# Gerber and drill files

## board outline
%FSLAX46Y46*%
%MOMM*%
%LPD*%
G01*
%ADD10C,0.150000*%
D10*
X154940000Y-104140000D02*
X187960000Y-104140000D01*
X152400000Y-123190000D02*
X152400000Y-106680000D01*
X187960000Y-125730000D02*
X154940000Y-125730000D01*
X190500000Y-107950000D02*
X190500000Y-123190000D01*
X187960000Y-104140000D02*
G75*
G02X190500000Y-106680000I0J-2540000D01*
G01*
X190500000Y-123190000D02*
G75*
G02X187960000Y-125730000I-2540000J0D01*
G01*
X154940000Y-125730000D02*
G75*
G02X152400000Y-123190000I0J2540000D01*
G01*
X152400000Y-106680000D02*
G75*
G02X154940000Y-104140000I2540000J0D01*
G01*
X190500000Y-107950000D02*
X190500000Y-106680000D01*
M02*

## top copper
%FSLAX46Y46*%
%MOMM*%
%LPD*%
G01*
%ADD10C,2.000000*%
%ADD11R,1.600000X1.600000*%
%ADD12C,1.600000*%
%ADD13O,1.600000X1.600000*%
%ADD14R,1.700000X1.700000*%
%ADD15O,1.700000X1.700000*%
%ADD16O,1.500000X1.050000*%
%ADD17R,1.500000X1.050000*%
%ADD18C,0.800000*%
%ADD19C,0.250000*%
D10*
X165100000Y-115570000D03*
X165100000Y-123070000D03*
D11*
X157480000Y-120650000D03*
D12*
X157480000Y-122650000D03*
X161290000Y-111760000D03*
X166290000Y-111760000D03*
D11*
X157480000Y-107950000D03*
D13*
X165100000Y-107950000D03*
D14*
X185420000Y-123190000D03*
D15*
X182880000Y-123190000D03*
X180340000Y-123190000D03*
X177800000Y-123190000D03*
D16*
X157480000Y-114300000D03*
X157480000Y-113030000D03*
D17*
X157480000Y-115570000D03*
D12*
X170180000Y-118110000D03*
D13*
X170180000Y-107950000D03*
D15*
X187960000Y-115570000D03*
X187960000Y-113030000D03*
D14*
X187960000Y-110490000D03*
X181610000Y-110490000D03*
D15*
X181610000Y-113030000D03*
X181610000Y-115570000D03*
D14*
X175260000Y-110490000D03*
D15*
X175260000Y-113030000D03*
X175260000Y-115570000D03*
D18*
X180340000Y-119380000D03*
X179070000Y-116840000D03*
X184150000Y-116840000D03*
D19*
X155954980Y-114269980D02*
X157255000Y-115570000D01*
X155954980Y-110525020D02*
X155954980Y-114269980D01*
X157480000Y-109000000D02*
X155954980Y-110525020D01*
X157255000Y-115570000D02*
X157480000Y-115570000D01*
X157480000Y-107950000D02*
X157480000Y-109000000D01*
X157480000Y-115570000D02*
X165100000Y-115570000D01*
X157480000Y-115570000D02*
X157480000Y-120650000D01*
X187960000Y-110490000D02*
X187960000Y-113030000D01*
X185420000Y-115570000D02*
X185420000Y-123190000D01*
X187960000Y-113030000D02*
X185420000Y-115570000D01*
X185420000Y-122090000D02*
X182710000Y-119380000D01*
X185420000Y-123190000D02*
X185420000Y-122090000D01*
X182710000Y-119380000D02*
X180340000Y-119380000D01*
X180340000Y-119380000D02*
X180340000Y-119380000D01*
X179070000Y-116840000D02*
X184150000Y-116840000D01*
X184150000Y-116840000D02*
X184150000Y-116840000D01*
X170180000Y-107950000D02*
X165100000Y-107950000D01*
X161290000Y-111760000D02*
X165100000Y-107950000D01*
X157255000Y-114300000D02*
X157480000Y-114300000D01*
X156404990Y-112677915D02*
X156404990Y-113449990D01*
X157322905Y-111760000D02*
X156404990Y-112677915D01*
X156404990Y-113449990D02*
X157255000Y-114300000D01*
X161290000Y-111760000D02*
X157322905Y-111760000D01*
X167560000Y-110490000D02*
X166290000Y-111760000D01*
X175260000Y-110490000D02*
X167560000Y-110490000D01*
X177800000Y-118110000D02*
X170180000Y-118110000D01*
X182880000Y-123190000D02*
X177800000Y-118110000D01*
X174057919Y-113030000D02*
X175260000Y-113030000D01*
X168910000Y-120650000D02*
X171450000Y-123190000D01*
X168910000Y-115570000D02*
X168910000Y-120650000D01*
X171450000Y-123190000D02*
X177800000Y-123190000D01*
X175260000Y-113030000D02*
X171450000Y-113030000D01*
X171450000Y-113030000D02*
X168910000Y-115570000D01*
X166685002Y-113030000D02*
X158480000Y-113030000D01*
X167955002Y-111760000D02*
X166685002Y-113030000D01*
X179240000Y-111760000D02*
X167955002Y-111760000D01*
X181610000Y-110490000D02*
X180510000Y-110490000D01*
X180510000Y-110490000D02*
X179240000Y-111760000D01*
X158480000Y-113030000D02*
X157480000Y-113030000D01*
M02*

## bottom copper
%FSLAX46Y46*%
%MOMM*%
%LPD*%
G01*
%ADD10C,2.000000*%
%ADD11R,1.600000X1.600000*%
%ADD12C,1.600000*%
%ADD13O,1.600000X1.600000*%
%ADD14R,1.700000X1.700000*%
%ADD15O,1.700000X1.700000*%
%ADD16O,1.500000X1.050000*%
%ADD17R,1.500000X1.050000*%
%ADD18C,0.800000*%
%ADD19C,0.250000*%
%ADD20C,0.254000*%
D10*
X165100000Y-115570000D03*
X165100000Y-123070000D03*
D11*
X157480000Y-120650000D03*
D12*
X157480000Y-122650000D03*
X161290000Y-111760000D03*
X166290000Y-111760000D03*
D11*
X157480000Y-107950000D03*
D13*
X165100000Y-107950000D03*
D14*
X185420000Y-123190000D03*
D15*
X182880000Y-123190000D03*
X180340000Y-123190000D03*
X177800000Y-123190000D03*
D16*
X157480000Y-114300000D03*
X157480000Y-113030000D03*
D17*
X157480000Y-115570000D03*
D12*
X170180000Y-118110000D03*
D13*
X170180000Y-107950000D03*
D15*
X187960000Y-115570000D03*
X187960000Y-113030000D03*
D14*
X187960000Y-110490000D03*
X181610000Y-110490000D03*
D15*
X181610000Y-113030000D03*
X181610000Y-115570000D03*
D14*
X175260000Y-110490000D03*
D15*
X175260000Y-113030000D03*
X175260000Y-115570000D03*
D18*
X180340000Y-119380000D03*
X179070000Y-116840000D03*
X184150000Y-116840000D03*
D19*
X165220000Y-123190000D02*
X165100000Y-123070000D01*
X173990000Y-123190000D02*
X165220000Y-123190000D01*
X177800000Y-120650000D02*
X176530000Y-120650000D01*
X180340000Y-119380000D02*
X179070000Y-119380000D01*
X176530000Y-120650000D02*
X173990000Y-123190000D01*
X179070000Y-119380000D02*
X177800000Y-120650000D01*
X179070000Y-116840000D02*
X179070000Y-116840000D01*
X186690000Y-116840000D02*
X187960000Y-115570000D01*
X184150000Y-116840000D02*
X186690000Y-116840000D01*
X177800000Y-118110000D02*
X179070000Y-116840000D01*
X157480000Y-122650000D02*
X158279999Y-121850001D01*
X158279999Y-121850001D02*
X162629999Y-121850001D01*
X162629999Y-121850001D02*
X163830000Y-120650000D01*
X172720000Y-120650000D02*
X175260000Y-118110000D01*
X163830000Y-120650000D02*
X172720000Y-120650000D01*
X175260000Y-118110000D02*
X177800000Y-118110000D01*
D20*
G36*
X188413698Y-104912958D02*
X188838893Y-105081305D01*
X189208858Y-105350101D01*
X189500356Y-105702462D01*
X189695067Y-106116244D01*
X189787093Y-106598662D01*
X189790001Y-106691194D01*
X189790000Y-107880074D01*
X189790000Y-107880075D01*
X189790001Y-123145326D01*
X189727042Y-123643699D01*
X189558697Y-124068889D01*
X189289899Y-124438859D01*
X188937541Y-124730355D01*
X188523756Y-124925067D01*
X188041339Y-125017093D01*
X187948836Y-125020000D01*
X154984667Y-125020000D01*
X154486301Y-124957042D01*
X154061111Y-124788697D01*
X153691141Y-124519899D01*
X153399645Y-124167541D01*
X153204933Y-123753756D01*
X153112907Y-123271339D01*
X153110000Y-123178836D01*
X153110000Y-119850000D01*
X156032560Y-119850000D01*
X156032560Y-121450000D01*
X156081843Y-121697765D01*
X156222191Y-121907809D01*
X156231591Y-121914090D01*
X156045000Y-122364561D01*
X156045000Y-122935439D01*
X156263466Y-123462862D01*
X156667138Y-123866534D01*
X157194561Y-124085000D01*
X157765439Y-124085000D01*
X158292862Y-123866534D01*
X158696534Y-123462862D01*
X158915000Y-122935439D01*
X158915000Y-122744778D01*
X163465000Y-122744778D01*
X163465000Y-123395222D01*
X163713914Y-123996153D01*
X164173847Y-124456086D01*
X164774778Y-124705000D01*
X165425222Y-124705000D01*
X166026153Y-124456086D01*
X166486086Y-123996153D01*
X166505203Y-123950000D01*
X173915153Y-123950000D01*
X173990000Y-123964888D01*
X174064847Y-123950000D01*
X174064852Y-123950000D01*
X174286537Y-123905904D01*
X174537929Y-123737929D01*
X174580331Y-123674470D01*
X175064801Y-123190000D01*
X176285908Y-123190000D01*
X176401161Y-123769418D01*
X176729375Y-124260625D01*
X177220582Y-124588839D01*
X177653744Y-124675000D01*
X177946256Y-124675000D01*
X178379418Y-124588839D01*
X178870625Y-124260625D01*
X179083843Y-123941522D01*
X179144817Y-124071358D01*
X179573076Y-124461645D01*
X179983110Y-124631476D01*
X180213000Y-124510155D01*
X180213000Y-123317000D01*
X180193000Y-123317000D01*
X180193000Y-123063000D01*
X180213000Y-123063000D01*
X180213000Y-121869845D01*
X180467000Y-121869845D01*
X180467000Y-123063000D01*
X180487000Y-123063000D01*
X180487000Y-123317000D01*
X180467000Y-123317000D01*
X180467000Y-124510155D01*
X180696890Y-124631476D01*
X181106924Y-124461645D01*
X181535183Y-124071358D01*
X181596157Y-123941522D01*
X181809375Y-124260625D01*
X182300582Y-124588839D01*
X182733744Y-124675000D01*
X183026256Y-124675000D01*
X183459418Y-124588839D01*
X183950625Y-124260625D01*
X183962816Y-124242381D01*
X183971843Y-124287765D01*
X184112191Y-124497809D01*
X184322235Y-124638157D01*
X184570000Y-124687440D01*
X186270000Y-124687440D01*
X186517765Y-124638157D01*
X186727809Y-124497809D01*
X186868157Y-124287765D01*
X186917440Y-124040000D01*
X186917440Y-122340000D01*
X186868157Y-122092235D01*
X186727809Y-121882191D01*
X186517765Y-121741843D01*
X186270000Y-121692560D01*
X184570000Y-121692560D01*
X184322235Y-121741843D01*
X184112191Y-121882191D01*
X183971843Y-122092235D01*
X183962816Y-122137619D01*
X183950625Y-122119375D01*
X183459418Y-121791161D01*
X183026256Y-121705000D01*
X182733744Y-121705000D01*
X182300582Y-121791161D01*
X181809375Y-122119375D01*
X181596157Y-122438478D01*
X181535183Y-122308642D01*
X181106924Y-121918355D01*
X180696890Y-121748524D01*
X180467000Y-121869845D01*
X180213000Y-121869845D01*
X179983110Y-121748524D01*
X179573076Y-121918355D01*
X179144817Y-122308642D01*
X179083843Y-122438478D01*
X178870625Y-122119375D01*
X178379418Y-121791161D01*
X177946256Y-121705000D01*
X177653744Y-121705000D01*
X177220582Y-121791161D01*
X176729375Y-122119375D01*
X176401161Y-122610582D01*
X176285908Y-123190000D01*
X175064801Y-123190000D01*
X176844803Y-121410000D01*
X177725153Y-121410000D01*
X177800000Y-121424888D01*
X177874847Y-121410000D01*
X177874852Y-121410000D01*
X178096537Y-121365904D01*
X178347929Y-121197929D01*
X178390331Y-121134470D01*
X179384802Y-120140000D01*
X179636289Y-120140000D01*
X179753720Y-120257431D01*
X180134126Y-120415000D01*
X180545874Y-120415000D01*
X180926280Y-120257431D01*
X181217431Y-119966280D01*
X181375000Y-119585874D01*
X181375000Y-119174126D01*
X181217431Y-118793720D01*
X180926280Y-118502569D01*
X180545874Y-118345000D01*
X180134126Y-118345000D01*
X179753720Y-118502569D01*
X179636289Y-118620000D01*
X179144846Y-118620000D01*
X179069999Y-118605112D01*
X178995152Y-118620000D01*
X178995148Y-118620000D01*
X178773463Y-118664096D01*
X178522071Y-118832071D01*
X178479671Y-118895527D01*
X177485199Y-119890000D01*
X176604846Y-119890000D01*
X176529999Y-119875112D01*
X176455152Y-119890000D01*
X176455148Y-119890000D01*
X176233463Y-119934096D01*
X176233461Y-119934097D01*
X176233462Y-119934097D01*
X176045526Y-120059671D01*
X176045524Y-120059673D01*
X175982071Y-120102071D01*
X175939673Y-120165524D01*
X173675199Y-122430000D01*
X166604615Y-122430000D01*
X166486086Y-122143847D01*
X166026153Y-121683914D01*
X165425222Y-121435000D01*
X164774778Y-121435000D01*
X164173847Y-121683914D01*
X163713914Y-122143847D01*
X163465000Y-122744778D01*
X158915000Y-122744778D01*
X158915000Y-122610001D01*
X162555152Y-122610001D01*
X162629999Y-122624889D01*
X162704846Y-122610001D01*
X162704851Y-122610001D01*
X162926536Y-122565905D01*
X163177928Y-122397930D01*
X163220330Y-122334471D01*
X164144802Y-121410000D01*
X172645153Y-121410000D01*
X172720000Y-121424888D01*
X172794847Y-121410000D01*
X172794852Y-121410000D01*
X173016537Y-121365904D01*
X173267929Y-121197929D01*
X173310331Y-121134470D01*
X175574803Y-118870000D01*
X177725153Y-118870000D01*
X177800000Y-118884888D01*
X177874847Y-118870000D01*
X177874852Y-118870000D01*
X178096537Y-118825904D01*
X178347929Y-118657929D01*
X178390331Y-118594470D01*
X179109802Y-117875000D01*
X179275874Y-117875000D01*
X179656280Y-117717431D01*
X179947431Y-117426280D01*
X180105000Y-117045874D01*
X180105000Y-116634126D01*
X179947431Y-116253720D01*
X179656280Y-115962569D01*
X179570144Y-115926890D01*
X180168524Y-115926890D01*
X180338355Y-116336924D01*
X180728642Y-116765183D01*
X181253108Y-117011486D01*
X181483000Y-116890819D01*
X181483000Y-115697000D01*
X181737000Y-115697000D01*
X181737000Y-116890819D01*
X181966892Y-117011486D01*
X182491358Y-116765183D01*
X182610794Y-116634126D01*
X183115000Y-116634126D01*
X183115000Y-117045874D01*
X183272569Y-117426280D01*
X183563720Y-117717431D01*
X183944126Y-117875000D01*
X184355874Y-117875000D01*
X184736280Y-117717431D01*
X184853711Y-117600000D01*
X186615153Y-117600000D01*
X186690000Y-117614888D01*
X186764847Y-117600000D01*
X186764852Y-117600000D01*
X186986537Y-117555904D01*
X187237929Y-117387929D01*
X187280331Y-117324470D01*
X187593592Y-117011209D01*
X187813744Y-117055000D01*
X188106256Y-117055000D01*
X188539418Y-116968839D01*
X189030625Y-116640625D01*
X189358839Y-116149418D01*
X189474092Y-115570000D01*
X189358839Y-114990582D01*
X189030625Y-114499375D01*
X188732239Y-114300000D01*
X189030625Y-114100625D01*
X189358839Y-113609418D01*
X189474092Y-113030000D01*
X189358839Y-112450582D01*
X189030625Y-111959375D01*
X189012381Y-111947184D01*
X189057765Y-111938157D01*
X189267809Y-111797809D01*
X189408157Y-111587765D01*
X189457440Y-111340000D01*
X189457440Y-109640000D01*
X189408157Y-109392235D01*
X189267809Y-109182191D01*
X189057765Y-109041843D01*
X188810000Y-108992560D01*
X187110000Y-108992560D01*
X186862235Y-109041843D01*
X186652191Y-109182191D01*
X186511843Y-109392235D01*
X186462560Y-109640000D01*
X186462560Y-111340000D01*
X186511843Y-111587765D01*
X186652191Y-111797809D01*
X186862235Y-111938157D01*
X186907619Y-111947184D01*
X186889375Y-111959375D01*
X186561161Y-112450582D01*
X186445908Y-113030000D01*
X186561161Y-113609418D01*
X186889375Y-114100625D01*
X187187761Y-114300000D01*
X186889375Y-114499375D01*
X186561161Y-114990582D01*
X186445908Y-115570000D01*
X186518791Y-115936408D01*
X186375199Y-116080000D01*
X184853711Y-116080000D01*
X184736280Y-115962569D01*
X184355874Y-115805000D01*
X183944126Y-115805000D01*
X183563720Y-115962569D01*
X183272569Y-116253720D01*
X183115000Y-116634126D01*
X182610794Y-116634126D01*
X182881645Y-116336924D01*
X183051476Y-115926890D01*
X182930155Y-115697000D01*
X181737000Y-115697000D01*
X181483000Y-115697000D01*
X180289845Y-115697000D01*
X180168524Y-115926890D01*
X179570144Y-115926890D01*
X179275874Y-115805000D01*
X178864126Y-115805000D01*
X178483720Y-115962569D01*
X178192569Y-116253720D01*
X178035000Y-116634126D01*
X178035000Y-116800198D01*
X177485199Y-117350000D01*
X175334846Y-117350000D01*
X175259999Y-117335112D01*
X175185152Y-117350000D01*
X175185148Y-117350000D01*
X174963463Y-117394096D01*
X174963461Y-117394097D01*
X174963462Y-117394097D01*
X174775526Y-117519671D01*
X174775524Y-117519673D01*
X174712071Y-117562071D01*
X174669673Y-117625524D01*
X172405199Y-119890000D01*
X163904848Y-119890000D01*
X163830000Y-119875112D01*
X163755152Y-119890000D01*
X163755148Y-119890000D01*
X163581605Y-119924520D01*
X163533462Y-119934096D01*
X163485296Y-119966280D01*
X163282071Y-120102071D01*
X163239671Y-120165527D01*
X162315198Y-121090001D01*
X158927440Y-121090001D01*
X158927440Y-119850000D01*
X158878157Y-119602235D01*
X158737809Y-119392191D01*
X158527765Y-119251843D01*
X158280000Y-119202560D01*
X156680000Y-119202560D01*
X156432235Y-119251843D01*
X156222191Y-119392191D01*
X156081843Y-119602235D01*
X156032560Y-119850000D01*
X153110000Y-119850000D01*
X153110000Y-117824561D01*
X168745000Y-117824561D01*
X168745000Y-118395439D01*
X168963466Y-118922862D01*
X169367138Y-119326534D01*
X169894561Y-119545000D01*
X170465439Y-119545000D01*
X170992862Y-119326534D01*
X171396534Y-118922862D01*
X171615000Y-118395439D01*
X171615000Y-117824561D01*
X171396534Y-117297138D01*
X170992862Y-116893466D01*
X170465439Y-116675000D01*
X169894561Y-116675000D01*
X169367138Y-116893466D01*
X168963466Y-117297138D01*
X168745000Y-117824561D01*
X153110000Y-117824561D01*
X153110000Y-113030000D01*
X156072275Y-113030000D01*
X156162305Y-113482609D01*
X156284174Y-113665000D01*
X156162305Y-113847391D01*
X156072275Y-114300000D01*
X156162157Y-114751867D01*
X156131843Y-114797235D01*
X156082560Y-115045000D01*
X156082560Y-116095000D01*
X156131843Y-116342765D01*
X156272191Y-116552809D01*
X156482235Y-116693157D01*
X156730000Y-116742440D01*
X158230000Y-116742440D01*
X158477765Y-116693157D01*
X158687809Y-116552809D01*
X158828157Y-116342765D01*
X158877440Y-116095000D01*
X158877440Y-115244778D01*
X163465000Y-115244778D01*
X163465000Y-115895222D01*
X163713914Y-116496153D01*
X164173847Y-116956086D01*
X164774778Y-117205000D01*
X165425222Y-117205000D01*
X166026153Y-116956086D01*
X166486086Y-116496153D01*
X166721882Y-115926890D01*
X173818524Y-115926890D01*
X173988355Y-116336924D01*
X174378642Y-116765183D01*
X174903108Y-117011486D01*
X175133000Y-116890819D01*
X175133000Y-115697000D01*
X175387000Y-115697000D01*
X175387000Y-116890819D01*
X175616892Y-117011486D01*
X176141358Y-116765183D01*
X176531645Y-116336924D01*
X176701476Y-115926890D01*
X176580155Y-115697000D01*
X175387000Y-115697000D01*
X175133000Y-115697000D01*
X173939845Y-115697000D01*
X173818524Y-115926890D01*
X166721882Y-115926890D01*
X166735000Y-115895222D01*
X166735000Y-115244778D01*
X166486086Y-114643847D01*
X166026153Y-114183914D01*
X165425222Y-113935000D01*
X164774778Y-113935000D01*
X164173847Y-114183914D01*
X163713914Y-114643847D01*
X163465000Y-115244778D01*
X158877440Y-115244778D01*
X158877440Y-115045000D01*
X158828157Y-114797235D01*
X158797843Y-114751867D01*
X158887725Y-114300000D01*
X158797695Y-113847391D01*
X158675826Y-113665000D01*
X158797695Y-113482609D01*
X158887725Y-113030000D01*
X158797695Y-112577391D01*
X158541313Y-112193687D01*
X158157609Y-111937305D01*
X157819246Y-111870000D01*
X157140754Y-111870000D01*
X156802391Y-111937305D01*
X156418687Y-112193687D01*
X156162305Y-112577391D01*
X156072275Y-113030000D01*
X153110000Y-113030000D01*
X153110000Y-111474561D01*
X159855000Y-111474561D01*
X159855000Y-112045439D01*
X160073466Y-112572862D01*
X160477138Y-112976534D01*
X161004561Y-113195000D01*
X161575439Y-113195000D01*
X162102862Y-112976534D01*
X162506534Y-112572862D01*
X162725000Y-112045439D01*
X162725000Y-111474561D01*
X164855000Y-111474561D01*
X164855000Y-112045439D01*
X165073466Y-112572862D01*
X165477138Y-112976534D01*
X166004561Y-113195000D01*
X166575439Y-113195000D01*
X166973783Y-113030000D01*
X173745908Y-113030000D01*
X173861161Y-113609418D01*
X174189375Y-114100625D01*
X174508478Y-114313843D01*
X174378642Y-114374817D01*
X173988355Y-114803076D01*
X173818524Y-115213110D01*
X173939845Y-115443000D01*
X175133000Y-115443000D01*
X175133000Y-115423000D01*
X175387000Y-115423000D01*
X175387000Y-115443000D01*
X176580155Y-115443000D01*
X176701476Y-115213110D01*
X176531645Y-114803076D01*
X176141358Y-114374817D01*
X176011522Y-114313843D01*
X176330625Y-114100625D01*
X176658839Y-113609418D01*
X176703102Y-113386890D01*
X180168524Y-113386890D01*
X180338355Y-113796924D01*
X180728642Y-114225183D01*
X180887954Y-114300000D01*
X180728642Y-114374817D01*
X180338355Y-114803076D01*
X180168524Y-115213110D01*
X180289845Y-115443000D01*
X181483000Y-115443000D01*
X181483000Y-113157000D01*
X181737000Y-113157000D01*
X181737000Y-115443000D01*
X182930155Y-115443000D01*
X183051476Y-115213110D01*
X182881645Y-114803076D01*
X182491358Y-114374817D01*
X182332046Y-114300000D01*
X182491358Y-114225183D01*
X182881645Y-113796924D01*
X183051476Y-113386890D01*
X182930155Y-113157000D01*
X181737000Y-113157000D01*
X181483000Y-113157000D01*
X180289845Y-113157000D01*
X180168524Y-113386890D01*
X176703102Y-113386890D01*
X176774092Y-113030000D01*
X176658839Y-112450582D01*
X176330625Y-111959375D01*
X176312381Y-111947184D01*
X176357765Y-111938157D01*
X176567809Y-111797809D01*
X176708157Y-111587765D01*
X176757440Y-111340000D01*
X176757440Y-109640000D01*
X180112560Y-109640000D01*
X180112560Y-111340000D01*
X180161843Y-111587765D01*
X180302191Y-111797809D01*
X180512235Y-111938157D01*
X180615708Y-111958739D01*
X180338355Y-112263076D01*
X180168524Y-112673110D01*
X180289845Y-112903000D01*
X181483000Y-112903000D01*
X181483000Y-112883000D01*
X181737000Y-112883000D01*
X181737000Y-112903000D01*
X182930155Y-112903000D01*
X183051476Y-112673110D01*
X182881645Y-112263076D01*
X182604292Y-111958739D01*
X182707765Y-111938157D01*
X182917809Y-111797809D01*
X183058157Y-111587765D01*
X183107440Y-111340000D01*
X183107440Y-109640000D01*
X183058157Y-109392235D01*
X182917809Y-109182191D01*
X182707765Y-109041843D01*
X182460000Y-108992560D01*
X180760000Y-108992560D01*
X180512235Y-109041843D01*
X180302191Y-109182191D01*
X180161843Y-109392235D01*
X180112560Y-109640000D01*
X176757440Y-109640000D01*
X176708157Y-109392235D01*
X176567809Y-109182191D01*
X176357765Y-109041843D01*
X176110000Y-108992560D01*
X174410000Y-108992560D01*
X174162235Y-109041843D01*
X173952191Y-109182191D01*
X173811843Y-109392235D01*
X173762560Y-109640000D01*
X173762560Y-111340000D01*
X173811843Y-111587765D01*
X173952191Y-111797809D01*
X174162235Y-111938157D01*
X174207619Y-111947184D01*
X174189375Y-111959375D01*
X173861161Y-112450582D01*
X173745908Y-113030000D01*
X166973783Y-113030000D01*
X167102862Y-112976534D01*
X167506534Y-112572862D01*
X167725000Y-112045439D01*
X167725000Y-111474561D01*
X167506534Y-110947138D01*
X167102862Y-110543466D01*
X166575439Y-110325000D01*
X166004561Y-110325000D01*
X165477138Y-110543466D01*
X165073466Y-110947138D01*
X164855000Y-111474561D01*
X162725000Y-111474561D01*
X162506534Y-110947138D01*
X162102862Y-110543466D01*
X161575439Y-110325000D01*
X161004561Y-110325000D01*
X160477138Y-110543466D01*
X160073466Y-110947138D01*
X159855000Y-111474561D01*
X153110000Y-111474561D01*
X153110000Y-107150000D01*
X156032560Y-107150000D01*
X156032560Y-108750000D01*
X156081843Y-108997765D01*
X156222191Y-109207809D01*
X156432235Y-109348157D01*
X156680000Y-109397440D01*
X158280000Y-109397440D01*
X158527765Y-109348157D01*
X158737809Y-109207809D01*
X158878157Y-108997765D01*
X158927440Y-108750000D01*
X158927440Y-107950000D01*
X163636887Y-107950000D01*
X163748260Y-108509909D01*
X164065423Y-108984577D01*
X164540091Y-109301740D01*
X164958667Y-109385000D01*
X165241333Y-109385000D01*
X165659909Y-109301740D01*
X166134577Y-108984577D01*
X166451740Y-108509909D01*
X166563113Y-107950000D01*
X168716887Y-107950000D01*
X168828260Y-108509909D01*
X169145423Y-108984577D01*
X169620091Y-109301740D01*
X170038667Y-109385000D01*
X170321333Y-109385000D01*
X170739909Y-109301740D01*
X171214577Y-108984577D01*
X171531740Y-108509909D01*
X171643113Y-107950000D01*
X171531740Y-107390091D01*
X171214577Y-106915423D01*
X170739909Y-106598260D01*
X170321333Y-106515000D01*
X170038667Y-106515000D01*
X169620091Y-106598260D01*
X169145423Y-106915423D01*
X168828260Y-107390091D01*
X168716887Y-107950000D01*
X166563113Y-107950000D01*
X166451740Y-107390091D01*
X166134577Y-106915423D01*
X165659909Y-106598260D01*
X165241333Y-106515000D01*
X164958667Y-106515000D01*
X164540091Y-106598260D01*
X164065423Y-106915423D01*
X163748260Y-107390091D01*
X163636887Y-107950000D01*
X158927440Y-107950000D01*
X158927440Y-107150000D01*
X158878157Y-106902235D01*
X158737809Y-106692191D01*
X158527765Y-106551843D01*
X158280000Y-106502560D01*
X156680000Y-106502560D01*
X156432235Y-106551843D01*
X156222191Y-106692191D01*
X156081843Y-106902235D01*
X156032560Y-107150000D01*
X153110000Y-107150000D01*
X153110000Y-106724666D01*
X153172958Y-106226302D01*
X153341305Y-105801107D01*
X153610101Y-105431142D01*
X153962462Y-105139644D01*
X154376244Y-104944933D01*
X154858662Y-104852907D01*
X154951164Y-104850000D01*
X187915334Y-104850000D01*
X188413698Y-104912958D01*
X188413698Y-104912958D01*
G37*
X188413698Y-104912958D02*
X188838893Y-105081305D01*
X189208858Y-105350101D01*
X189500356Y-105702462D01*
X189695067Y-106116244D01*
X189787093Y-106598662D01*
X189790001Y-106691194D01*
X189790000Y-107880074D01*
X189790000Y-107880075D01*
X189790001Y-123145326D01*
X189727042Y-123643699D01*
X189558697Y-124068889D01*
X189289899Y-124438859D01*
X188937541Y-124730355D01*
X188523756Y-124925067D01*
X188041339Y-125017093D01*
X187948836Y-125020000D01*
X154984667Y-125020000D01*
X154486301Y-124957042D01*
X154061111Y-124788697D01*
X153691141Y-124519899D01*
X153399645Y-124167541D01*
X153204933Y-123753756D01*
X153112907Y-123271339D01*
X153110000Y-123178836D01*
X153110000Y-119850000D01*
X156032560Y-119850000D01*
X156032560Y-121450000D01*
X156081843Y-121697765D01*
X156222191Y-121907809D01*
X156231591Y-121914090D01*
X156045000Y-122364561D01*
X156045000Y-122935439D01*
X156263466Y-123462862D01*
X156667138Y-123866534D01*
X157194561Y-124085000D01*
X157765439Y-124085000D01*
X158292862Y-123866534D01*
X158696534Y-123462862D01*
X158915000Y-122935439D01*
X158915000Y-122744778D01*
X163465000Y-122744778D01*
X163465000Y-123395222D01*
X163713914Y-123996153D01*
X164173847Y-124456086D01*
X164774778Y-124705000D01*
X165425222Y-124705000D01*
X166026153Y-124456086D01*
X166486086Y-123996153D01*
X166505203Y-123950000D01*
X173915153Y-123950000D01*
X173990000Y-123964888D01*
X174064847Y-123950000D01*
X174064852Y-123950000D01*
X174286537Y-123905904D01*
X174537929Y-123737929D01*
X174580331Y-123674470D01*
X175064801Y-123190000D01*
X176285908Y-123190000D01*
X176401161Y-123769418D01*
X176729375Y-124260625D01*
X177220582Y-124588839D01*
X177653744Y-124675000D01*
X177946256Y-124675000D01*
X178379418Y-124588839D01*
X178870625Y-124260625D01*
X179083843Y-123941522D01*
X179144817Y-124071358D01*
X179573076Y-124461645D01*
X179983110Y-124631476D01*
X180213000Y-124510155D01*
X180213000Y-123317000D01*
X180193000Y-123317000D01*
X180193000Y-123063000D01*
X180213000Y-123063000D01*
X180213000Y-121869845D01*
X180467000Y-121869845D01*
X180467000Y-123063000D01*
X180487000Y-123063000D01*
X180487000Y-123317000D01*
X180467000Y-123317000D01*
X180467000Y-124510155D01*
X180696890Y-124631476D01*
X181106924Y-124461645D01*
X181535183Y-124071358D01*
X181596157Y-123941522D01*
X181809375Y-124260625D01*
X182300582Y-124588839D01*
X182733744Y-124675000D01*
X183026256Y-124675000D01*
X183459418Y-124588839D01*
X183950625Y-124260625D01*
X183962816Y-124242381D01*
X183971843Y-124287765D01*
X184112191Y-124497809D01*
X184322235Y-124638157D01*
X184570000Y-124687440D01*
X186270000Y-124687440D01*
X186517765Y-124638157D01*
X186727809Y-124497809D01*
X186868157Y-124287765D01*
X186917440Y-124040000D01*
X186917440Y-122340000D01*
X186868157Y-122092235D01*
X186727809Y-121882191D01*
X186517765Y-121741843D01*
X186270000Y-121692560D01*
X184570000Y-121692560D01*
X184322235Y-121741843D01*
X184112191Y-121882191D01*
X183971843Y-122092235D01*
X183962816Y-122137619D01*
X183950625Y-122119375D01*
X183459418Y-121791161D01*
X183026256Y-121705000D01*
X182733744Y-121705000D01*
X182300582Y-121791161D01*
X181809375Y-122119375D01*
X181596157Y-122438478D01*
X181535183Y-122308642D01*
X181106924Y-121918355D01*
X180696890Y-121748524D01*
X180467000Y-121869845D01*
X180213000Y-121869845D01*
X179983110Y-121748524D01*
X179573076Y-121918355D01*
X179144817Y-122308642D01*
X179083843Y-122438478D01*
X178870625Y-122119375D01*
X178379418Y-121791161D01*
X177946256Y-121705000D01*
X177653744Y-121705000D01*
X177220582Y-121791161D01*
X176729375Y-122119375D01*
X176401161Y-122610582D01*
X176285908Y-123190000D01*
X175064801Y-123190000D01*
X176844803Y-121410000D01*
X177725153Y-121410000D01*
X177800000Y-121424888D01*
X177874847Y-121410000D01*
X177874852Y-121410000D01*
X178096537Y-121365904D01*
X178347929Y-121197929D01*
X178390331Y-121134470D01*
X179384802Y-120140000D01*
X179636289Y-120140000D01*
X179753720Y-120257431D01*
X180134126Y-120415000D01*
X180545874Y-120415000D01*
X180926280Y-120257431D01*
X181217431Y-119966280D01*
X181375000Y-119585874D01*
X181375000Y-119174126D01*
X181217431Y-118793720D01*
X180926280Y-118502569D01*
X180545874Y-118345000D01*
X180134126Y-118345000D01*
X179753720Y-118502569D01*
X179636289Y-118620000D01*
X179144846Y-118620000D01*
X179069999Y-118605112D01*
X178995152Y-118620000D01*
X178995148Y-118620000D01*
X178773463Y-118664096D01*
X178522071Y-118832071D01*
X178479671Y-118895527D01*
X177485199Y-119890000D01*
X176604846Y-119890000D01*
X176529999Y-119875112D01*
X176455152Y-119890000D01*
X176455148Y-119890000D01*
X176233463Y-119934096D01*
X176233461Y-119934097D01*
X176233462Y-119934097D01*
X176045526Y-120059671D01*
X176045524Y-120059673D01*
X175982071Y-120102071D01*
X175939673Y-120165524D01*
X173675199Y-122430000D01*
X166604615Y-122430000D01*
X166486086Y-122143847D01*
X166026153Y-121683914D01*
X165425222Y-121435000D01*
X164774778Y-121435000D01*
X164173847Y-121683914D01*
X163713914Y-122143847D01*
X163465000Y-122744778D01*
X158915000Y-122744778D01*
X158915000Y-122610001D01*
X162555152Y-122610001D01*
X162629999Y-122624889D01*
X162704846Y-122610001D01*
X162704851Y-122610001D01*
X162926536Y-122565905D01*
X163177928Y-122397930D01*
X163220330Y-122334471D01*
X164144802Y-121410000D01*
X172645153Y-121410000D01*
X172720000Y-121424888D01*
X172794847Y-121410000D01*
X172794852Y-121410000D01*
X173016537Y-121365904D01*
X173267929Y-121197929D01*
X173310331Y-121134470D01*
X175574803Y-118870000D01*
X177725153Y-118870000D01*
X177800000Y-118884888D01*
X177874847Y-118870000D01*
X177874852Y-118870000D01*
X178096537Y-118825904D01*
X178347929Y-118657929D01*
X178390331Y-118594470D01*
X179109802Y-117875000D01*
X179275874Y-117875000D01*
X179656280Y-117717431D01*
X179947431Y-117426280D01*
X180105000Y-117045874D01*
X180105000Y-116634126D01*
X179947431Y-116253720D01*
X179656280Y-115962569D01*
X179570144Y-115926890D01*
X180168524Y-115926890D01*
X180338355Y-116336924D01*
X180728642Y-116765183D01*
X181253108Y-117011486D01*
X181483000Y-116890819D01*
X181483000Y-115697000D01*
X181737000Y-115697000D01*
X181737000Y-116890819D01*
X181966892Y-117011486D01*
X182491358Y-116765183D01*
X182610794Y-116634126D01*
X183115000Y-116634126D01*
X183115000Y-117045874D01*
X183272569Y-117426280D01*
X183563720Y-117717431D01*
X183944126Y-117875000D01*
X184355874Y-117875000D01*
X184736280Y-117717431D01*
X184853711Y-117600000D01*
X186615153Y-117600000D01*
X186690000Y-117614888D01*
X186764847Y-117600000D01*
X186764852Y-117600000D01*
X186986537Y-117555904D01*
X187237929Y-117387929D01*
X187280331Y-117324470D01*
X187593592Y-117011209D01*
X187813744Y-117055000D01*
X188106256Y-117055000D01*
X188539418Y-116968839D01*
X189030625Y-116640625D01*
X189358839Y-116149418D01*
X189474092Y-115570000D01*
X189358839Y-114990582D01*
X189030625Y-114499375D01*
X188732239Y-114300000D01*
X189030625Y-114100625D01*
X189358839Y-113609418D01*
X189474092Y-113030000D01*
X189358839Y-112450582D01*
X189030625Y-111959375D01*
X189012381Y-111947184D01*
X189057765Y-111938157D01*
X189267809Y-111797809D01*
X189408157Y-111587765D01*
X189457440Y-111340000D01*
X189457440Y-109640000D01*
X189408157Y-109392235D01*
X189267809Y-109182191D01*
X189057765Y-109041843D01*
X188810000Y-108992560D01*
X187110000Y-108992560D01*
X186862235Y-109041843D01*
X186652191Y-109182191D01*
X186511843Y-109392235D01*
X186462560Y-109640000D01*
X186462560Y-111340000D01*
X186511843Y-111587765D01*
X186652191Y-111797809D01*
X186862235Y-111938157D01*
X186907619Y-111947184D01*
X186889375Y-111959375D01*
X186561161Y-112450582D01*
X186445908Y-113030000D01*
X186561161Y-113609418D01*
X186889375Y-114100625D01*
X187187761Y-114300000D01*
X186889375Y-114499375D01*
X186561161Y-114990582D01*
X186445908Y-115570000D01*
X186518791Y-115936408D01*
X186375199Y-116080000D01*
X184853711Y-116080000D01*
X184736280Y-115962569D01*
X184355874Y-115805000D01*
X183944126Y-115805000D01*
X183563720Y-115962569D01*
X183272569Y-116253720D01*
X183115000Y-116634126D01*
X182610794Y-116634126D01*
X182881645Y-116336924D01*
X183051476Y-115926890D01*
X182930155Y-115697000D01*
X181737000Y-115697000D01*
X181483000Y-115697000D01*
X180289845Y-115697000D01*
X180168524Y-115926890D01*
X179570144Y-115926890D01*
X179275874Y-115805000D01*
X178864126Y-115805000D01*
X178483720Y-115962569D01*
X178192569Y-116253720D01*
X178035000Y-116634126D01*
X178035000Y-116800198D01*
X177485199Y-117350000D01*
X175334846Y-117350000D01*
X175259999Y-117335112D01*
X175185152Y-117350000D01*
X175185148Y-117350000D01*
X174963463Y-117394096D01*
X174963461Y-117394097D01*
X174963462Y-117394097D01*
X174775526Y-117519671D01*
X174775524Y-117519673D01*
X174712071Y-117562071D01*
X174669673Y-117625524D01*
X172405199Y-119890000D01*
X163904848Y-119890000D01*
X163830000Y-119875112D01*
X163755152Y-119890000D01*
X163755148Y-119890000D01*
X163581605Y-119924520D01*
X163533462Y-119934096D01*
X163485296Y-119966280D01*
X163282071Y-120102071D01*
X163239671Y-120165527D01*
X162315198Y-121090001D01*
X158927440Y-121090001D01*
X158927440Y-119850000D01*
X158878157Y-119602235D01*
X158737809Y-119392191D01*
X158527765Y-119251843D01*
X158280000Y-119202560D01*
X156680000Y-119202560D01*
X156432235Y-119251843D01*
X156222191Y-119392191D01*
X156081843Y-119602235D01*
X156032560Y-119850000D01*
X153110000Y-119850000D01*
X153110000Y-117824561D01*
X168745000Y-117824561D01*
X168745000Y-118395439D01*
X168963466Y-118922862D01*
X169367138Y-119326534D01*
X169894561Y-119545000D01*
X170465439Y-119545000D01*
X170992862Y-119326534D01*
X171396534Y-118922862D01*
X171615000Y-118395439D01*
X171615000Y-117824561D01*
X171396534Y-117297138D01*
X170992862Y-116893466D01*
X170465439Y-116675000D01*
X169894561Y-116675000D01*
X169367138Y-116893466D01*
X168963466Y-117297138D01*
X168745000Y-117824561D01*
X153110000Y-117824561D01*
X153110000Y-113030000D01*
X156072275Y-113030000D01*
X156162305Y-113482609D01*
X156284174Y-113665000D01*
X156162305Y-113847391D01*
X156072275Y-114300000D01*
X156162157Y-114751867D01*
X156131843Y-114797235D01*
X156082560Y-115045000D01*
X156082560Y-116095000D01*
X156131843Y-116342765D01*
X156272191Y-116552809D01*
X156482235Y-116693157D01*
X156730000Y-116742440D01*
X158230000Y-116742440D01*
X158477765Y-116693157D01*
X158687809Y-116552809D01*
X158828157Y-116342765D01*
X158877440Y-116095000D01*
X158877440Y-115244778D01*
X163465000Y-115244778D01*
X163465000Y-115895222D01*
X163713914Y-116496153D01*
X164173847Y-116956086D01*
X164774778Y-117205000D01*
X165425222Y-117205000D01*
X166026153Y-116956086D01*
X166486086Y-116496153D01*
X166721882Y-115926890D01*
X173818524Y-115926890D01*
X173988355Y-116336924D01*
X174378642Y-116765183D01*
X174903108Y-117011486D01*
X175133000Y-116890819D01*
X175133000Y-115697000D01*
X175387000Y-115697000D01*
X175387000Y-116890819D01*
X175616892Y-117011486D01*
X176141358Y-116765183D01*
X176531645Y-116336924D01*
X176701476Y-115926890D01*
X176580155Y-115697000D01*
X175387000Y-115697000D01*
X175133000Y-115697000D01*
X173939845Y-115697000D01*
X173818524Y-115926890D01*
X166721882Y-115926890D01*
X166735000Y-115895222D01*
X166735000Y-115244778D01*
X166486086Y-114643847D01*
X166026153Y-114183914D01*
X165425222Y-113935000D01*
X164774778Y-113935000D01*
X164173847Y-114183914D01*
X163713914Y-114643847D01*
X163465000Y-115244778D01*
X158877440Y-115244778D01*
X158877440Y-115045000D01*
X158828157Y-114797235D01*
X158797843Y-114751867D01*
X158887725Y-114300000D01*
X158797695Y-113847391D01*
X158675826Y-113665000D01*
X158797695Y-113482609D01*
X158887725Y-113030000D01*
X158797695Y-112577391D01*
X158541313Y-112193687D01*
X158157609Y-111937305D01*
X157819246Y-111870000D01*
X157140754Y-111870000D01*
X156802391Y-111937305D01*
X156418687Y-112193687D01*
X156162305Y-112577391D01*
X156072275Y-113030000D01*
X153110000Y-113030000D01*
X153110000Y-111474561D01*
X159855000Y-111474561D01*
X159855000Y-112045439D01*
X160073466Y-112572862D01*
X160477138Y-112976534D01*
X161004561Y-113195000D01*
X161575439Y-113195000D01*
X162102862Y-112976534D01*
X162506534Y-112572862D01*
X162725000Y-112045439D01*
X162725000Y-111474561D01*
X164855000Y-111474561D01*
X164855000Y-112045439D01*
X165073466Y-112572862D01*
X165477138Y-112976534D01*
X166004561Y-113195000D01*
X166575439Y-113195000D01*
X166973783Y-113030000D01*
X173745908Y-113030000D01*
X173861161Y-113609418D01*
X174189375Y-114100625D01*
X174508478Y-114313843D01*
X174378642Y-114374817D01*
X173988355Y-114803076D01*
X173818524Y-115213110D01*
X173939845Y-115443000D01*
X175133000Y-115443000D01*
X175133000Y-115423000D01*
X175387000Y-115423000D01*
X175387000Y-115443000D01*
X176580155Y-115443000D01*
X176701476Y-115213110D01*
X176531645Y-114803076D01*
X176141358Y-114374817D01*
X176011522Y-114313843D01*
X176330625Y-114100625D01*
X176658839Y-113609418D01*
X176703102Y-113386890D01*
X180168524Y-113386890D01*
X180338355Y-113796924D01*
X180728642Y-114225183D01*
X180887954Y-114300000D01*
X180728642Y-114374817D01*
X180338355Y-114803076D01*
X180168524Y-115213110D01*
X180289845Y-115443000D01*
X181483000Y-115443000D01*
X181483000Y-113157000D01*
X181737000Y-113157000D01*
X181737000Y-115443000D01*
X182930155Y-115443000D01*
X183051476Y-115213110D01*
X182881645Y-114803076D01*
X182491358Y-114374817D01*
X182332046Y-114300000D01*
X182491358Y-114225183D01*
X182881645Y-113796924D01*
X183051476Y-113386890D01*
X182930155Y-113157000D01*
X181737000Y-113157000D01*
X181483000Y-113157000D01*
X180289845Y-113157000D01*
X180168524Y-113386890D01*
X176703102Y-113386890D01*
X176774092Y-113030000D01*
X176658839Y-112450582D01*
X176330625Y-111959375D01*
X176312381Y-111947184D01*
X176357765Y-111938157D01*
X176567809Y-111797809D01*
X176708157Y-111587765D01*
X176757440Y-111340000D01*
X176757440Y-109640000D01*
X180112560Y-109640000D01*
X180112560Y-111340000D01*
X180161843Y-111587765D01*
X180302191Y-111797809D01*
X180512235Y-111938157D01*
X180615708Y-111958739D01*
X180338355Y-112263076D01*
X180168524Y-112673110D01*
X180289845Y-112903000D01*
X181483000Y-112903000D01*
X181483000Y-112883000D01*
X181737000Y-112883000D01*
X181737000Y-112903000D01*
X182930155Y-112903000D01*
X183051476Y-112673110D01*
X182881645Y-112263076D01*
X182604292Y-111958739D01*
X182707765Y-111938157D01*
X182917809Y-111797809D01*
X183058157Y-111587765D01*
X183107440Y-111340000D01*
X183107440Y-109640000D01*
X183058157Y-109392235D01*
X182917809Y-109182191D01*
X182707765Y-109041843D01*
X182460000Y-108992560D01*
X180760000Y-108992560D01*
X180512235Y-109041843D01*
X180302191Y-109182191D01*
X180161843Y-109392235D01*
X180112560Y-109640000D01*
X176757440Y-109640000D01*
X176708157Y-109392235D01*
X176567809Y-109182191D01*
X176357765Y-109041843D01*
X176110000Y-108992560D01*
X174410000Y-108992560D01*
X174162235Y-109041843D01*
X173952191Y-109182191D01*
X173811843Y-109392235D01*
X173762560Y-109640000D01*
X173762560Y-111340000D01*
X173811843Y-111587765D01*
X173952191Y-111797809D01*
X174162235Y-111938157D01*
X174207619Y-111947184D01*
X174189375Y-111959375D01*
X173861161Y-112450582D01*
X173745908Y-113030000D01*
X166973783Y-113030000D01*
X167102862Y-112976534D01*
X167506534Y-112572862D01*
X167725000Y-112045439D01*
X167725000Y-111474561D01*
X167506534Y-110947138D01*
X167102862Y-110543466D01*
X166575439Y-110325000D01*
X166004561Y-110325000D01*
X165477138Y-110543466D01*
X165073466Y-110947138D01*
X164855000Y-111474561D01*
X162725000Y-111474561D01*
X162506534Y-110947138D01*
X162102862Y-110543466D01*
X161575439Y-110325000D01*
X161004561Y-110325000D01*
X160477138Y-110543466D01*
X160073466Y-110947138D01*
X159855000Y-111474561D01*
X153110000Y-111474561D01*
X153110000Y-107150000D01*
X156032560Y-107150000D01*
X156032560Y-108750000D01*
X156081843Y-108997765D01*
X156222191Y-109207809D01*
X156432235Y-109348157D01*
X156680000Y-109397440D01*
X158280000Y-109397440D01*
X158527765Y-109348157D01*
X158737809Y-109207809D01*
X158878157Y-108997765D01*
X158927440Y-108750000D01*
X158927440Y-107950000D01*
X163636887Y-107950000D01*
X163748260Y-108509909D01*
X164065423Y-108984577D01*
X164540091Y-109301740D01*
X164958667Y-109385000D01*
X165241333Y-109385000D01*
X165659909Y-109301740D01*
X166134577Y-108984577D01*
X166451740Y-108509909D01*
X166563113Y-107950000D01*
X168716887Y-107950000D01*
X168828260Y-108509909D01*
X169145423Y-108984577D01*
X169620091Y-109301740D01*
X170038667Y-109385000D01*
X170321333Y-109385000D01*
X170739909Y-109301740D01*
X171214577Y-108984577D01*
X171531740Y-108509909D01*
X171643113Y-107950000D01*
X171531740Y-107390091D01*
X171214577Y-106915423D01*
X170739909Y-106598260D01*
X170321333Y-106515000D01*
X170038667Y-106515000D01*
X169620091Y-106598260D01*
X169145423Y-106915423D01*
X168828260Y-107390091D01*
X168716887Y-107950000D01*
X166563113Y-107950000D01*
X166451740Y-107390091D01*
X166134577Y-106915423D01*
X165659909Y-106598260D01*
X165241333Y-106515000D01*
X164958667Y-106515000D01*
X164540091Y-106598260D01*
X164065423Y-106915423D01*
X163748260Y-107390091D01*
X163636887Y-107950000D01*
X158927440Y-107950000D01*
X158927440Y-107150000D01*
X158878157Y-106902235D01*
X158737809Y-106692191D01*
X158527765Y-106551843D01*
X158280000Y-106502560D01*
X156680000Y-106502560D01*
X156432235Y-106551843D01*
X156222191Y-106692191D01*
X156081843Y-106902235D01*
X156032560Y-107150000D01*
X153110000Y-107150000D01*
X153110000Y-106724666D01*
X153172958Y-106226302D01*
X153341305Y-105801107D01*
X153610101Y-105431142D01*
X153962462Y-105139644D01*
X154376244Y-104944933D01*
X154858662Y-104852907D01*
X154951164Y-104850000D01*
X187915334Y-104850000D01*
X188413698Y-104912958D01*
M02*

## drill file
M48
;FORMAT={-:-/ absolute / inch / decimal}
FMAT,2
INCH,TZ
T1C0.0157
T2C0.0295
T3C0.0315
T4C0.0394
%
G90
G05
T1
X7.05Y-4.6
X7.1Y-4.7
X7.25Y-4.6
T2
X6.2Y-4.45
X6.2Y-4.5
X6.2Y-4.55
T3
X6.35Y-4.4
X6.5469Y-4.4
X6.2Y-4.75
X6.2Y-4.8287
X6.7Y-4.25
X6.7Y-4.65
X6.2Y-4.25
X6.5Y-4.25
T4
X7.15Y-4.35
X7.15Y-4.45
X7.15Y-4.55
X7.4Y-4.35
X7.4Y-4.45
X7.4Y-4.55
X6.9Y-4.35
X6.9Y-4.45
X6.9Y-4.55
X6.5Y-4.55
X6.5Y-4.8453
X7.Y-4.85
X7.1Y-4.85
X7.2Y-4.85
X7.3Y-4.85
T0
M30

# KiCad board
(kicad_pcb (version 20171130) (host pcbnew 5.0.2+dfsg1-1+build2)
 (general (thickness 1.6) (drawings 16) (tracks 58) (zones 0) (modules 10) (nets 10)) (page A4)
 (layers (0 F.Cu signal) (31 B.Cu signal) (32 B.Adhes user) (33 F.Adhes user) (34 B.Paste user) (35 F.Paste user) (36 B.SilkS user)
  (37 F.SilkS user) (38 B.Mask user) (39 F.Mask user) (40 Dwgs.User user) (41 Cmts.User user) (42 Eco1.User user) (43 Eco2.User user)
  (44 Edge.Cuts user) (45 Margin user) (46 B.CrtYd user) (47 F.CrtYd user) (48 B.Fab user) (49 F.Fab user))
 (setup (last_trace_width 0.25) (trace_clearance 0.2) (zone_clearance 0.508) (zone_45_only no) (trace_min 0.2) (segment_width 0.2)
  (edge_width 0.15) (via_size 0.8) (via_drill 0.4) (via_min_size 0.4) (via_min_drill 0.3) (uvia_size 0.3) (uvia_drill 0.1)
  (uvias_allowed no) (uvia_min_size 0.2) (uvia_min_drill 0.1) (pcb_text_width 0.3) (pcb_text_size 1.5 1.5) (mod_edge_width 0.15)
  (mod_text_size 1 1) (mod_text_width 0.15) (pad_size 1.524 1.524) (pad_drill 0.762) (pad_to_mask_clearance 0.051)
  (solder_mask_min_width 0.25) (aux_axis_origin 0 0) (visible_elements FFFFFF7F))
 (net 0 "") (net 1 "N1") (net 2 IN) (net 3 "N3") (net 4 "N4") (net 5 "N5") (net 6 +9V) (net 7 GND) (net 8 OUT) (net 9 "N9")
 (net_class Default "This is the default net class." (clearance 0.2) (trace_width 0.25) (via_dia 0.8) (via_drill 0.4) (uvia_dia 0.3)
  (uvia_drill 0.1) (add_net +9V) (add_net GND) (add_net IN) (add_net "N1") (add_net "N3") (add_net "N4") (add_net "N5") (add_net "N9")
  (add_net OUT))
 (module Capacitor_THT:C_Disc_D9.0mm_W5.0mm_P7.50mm (layer F.Cu) (at 165.1 115.57 270)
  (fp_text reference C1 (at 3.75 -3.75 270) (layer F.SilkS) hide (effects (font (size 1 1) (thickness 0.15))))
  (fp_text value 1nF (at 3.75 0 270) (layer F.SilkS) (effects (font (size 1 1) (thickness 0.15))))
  (pad 1 thru_hole circle (at 0 0 270) (size 2 2) (drill 1) (layers *.Cu *.Mask) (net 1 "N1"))
  (pad 2 thru_hole circle (at 7.5 0 270) (size 2 2) (drill 1) (layers *.Cu *.Mask) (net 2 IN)))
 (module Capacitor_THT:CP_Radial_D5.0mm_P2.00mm (layer F.Cu) (at 157.48 120.65 270)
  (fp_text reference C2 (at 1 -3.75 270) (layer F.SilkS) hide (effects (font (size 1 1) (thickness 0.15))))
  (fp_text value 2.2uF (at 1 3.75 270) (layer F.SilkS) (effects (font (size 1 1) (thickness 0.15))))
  (pad 1 thru_hole rect (at 0 0 270) (size 1.6 1.6) (drill 0.8) (layers *.Cu *.Mask) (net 1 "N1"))
  (pad 2 thru_hole circle (at 2 0 270) (size 1.6 1.6) (drill 0.8) (layers *.Cu *.Mask) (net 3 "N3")))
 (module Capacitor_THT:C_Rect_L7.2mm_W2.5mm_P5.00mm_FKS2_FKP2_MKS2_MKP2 (layer F.Cu) (at 161.29 111.76)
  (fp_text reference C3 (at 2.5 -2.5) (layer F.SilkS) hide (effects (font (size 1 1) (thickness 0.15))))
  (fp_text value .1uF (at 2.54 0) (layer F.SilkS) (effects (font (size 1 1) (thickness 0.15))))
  (pad 1 thru_hole circle (at 0 0) (size 1.6 1.6) (drill 0.8) (layers *.Cu *.Mask) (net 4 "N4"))
  (pad 2 thru_hole circle (at 5 0) (size 1.6 1.6) (drill 0.8) (layers *.Cu *.Mask) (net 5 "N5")))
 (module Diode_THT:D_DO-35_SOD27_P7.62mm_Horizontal (layer F.Cu) (at 157.48 107.95)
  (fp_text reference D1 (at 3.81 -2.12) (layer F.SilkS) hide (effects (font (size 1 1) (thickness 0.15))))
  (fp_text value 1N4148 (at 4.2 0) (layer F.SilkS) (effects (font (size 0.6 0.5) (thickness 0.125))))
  (pad 1 thru_hole rect (at 0 0) (size 1.6 1.6) (drill 0.8) (layers *.Cu *.Mask) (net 1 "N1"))
  (pad 2 thru_hole oval (at 7.62 0) (size 1.6 1.6) (drill 0.8) (layers *.Cu *.Mask) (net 4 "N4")))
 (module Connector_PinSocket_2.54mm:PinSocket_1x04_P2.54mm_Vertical (layer F.Cu) (at 185.42 123.19 270)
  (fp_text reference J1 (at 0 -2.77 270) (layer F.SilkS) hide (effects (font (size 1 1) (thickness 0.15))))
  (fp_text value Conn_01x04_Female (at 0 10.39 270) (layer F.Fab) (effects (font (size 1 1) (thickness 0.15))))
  (pad 1 thru_hole rect (at 0 0 270) (size 1.7 1.7) (drill 1) (layers *.Cu *.Mask) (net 2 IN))
  (pad 2 thru_hole oval (at 0 2.54 270) (size 1.7 1.7) (drill 1) (layers *.Cu *.Mask) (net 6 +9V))
  (pad 3 thru_hole oval (at 0 5.08 270) (size 1.7 1.7) (drill 1) (layers *.Cu *.Mask) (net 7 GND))
  (pad 4 thru_hole oval (at 0 7.62 270) (size 1.7 1.7) (drill 1) (layers *.Cu *.Mask) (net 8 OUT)))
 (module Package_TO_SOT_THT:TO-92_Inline (layer F.Cu) (at 157.48 115.57 90)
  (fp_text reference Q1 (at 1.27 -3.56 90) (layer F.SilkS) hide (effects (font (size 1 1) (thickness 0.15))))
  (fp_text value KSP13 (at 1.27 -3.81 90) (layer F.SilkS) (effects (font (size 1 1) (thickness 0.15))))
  (pad 2 thru_hole oval (at 1.27 0 90) (size 1.05 1.5) (drill 0.75) (layers *.Cu *.Mask) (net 4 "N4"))
  (pad 3 thru_hole oval (at 2.54 0 90) (size 1.05 1.5) (drill 0.75) (layers *.Cu *.Mask) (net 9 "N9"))
  (pad 1 thru_hole rect (at 0 0 90) (size 1.05 1.5) (drill 0.75) (layers *.Cu *.Mask) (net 1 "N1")))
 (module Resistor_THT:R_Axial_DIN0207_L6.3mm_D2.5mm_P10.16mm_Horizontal (layer F.Cu) (at 170.18 118.11 90)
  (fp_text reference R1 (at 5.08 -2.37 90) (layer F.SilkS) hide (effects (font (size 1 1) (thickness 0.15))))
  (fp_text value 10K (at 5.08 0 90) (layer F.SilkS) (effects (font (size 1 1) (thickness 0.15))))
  (pad 1 thru_hole circle (at 0 0 90) (size 1.6 1.6) (drill 0.8) (layers *.Cu *.Mask) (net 6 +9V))
  (pad 2 thru_hole oval (at 10.16 0 90) (size 1.6 1.6) (drill 0.8) (layers *.Cu *.Mask) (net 4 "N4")))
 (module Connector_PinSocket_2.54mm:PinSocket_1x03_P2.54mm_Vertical (layer F.Cu) (at 187.96 110.49)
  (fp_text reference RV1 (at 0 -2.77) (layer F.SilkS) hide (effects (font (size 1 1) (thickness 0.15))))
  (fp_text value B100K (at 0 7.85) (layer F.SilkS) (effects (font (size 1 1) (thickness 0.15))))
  (pad 3 thru_hole oval (at 0 5.08) (size 1.7 1.7) (drill 1) (layers *.Cu *.Mask) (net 3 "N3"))
  (pad 2 thru_hole oval (at 0 2.54) (size 1.7 1.7) (drill 1) (layers *.Cu *.Mask) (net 2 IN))
  (pad 1 thru_hole rect (at 0 0) (size 1.7 1.7) (drill 1) (layers *.Cu *.Mask) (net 2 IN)))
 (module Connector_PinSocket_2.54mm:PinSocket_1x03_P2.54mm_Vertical (layer F.Cu) (at 181.61 110.49)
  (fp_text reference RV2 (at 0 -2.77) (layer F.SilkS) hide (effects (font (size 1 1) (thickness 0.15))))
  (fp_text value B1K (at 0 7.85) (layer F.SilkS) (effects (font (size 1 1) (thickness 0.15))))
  (pad 1 thru_hole rect (at 0 0) (size 1.7 1.7) (drill 1) (layers *.Cu *.Mask) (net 9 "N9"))
  (pad 2 thru_hole oval (at 0 2.54) (size 1.7 1.7) (drill 1) (layers *.Cu *.Mask) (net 7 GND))
  (pad 3 thru_hole oval (at 0 5.08) (size 1.7 1.7) (drill 1) (layers *.Cu *.Mask) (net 7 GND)))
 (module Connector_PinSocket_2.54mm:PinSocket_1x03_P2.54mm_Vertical (layer F.Cu) (at 175.26 110.49)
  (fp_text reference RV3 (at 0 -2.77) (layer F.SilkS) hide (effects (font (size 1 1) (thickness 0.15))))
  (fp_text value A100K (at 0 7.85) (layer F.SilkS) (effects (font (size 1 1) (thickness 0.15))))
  (pad 1 thru_hole rect (at 0 0) (size 1.7 1.7) (drill 1) (layers *.Cu *.Mask) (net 5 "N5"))
  (pad 2 thru_hole oval (at 0 2.54) (size 1.7 1.7) (drill 1) (layers *.Cu *.Mask) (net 8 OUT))
  (pad 3 thru_hole oval (at 0 5.08) (size 1.7 1.7) (drill 1) (layers *.Cu *.Mask) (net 7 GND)))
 (gr_line (start 154.94 104.14) (end 187.96 104.14) (layer Edge.Cuts) (width 0.15))
 (gr_line (start 152.4 123.19) (end 152.4 106.68) (layer Edge.Cuts) (width 0.15))
 (gr_line (start 187.96 125.73) (end 154.94 125.73) (layer Edge.Cuts) (width 0.15))
 (gr_line (start 190.5 107.95) (end 190.5 123.19) (layer Edge.Cuts) (width 0.15))
 (gr_arc (start 187.96 106.68) (end 190.5 106.68) (angle -90) (layer Edge.Cuts) (width 0.15))
 (gr_arc (start 187.96 123.19) (end 187.96 125.73) (angle -90) (layer Edge.Cuts) (width 0.15))
 (gr_arc (start 154.94 123.19) (end 152.4 123.19) (angle -90) (layer Edge.Cuts) (width 0.15))
 (gr_arc (start 154.94 106.68) (end 154.94 104.14) (angle -90) (layer Edge.Cuts) (width 0.15))
 (gr_line (start 190.5 107.95) (end 190.5 106.68) (layer Edge.Cuts) (width 0.15))
 (segment (start 155.95498 114.26998) (end 157.255 115.57) (width 0.25) (layer F.Cu) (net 1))
 (segment (start 155.95498 110.52502) (end 155.95498 114.26998) (width 0.25) (layer F.Cu) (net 1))
 (segment (start 157.48 109) (end 155.95498 110.52502) (width 0.25) (layer F.Cu) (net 1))
 (segment (start 157.255 115.57) (end 157.48 115.57) (width 0.25) (layer F.Cu) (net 1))
 (segment (start 157.48 107.95) (end 157.48 109) (width 0.25) (layer F.Cu) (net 1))
 (segment (start 157.48 115.57) (end 165.1 115.57) (width 0.25) (layer F.Cu) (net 1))
 (segment (start 157.48 115.57) (end 157.48 120.65) (width 0.25) (layer F.Cu) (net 1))
 (segment (start 187.96 110.49) (end 187.96 113.03) (width 0.25) (layer F.Cu) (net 2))
 (segment (start 185.42 115.57) (end 185.42 123.19) (width 0.25) (layer F.Cu) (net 2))
 (segment (start 187.96 113.03) (end 185.42 115.57) (width 0.25) (layer F.Cu) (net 2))
 (segment (start 185.42 122.09) (end 182.71 119.38) (width 0.25) (layer F.Cu) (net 2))
 (segment (start 185.42 123.19) (end 185.42 122.09) (width 0.25) (layer F.Cu) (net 2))
 (segment (start 182.71 119.38) (end 180.34 119.38) (width 0.25) (layer F.Cu) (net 2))
 (segment (start 180.34 119.38) (end 180.34 119.38) (width 0.25) (layer F.Cu) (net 2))
 (via (at 180.34 119.38) (size 0.8) (drill 0.4) (layers F.Cu B.Cu) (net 2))
 (segment (start 165.22 123.19) (end 165.1 123.07) (width 0.25) (layer B.Cu) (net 2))
 (segment (start 173.99 123.19) (end 165.22 123.19) (width 0.25) (layer B.Cu) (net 2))
 (segment (start 177.8 120.65) (end 176.53 120.65) (width 0.25) (layer B.Cu) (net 2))
 (segment (start 180.34 119.38) (end 179.07 119.38) (width 0.25) (layer B.Cu) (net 2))
 (segment (start 176.53 120.65) (end 173.99 123.19) (width 0.25) (layer B.Cu) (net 2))
 (segment (start 179.07 119.38) (end 177.8 120.65) (width 0.25) (layer B.Cu) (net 2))
 (segment (start 179.07 116.84) (end 179.07 116.84) (width 0.25) (layer B.Cu) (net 3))
 (via (at 179.07 116.84) (size 0.8) (drill 0.4) (layers F.Cu B.Cu) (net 3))
 (segment (start 179.07 116.84) (end 184.15 116.84) (width 0.25) (layer F.Cu) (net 3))
 (segment (start 184.15 116.84) (end 184.15 116.84) (width 0.25) (layer F.Cu) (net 3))
 (via (at 184.15 116.84) (size 0.8) (drill 0.4) (layers F.Cu B.Cu) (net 3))
 (segment (start 186.69 116.84) (end 187.96 115.57) (width 0.25) (layer B.Cu) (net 3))
 (segment (start 184.15 116.84) (end 186.69 116.84) (width 0.25) (layer B.Cu) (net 3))
 (segment (start 177.8 118.11) (end 179.07 116.84) (width 0.25) (layer B.Cu) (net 3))
 (segment (start 157.48 122.65) (end 158.279999 121.850001) (width 0.25) (layer B.Cu) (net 3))
 (segment (start 158.279999 121.850001) (end 162.629999 121.850001) (width 0.25) (layer B.Cu) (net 3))
 (segment (start 162.629999 121.850001) (end 163.83 120.65) (width 0.25) (layer B.Cu) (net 3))
 (segment (start 172.72 120.65) (end 175.26 118.11) (width 0.25) (layer B.Cu) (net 3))
 (segment (start 163.83 120.65) (end 172.72 120.65) (width 0.25) (layer B.Cu) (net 3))
 (segment (start 175.26 118.11) (end 177.8 118.11) (width 0.25) (layer B.Cu) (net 3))
 (segment (start 170.18 107.95) (end 165.1 107.95) (width 0.25) (layer F.Cu) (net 4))
 (segment (start 161.29 111.76) (end 165.1 107.95) (width 0.25) (layer F.Cu) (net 4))
 (segment (start 157.255 114.3) (end 157.48 114.3) (width 0.25) (layer F.Cu) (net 4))
 (segment (start 156.40499 112.677915) (end 156.40499 113.44999) (width 0.25) (layer F.Cu) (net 4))
 (segment (start 157.322905 111.76) (end 156.40499 112.677915) (width 0.25) (layer F.Cu) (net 4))
 (segment (start 156.40499 113.44999) (end 157.255 114.3) (width 0.25) (layer F.Cu) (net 4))
 (segment (start 161.29 111.76) (end 157.322905 111.76) (width 0.25) (layer F.Cu) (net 4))
 (segment (start 167.56 110.49) (end 166.29 111.76) (width 0.25) (layer F.Cu) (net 5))
 (segment (start 175.26 110.49) (end 167.56 110.49) (width 0.25) (layer F.Cu) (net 5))
 (segment (start 177.8 118.11) (end 170.18 118.11) (width 0.25) (layer F.Cu) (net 6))
 (segment (start 182.88 123.19) (end 177.8 118.11) (width 0.25) (layer F.Cu) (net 6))
 (segment (start 174.057919 113.03) (end 175.26 113.03) (width 0.25) (layer F.Cu) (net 8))
 (segment (start 168.91 120.65) (end 171.45 123.19) (width 0.25) (layer F.Cu) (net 8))
 (segment (start 168.91 115.57) (end 168.91 120.65) (width 0.25) (layer F.Cu) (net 8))
 (segment (start 171.45 123.19) (end 177.8 123.19) (width 0.25) (layer F.Cu) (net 8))
 (segment (start 175.26 113.03) (end 171.45 113.03) (width 0.25) (layer F.Cu) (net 8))
 (segment (start 171.45 113.03) (end 168.91 115.57) (width 0.25) (layer F.Cu) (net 8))
 (segment (start 166.685002 113.03) (end 158.48 113.03) (width 0.25) (layer F.Cu) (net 9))
 (segment (start 167.955002 111.76) (end 166.685002 113.03) (width 0.25) (layer F.Cu) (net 9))
 (segment (start 179.24 111.76) (end 167.955002 111.76) (width 0.25) (layer F.Cu) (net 9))
 (segment (start 181.61 110.49) (end 180.51 110.49) (width 0.25) (layer F.Cu) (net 9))
 (segment (start 180.51 110.49) (end 179.24 111.76) (width 0.25) (layer F.Cu) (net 9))
 (segment (start 158.48 113.03) (end 157.48 113.03) (width 0.25) (layer F.Cu) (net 9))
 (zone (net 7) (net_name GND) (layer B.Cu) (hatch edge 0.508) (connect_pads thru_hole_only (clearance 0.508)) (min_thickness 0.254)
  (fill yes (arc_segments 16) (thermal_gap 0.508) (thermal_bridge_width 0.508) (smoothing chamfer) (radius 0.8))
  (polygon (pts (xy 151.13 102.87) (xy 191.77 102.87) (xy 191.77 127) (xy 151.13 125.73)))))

